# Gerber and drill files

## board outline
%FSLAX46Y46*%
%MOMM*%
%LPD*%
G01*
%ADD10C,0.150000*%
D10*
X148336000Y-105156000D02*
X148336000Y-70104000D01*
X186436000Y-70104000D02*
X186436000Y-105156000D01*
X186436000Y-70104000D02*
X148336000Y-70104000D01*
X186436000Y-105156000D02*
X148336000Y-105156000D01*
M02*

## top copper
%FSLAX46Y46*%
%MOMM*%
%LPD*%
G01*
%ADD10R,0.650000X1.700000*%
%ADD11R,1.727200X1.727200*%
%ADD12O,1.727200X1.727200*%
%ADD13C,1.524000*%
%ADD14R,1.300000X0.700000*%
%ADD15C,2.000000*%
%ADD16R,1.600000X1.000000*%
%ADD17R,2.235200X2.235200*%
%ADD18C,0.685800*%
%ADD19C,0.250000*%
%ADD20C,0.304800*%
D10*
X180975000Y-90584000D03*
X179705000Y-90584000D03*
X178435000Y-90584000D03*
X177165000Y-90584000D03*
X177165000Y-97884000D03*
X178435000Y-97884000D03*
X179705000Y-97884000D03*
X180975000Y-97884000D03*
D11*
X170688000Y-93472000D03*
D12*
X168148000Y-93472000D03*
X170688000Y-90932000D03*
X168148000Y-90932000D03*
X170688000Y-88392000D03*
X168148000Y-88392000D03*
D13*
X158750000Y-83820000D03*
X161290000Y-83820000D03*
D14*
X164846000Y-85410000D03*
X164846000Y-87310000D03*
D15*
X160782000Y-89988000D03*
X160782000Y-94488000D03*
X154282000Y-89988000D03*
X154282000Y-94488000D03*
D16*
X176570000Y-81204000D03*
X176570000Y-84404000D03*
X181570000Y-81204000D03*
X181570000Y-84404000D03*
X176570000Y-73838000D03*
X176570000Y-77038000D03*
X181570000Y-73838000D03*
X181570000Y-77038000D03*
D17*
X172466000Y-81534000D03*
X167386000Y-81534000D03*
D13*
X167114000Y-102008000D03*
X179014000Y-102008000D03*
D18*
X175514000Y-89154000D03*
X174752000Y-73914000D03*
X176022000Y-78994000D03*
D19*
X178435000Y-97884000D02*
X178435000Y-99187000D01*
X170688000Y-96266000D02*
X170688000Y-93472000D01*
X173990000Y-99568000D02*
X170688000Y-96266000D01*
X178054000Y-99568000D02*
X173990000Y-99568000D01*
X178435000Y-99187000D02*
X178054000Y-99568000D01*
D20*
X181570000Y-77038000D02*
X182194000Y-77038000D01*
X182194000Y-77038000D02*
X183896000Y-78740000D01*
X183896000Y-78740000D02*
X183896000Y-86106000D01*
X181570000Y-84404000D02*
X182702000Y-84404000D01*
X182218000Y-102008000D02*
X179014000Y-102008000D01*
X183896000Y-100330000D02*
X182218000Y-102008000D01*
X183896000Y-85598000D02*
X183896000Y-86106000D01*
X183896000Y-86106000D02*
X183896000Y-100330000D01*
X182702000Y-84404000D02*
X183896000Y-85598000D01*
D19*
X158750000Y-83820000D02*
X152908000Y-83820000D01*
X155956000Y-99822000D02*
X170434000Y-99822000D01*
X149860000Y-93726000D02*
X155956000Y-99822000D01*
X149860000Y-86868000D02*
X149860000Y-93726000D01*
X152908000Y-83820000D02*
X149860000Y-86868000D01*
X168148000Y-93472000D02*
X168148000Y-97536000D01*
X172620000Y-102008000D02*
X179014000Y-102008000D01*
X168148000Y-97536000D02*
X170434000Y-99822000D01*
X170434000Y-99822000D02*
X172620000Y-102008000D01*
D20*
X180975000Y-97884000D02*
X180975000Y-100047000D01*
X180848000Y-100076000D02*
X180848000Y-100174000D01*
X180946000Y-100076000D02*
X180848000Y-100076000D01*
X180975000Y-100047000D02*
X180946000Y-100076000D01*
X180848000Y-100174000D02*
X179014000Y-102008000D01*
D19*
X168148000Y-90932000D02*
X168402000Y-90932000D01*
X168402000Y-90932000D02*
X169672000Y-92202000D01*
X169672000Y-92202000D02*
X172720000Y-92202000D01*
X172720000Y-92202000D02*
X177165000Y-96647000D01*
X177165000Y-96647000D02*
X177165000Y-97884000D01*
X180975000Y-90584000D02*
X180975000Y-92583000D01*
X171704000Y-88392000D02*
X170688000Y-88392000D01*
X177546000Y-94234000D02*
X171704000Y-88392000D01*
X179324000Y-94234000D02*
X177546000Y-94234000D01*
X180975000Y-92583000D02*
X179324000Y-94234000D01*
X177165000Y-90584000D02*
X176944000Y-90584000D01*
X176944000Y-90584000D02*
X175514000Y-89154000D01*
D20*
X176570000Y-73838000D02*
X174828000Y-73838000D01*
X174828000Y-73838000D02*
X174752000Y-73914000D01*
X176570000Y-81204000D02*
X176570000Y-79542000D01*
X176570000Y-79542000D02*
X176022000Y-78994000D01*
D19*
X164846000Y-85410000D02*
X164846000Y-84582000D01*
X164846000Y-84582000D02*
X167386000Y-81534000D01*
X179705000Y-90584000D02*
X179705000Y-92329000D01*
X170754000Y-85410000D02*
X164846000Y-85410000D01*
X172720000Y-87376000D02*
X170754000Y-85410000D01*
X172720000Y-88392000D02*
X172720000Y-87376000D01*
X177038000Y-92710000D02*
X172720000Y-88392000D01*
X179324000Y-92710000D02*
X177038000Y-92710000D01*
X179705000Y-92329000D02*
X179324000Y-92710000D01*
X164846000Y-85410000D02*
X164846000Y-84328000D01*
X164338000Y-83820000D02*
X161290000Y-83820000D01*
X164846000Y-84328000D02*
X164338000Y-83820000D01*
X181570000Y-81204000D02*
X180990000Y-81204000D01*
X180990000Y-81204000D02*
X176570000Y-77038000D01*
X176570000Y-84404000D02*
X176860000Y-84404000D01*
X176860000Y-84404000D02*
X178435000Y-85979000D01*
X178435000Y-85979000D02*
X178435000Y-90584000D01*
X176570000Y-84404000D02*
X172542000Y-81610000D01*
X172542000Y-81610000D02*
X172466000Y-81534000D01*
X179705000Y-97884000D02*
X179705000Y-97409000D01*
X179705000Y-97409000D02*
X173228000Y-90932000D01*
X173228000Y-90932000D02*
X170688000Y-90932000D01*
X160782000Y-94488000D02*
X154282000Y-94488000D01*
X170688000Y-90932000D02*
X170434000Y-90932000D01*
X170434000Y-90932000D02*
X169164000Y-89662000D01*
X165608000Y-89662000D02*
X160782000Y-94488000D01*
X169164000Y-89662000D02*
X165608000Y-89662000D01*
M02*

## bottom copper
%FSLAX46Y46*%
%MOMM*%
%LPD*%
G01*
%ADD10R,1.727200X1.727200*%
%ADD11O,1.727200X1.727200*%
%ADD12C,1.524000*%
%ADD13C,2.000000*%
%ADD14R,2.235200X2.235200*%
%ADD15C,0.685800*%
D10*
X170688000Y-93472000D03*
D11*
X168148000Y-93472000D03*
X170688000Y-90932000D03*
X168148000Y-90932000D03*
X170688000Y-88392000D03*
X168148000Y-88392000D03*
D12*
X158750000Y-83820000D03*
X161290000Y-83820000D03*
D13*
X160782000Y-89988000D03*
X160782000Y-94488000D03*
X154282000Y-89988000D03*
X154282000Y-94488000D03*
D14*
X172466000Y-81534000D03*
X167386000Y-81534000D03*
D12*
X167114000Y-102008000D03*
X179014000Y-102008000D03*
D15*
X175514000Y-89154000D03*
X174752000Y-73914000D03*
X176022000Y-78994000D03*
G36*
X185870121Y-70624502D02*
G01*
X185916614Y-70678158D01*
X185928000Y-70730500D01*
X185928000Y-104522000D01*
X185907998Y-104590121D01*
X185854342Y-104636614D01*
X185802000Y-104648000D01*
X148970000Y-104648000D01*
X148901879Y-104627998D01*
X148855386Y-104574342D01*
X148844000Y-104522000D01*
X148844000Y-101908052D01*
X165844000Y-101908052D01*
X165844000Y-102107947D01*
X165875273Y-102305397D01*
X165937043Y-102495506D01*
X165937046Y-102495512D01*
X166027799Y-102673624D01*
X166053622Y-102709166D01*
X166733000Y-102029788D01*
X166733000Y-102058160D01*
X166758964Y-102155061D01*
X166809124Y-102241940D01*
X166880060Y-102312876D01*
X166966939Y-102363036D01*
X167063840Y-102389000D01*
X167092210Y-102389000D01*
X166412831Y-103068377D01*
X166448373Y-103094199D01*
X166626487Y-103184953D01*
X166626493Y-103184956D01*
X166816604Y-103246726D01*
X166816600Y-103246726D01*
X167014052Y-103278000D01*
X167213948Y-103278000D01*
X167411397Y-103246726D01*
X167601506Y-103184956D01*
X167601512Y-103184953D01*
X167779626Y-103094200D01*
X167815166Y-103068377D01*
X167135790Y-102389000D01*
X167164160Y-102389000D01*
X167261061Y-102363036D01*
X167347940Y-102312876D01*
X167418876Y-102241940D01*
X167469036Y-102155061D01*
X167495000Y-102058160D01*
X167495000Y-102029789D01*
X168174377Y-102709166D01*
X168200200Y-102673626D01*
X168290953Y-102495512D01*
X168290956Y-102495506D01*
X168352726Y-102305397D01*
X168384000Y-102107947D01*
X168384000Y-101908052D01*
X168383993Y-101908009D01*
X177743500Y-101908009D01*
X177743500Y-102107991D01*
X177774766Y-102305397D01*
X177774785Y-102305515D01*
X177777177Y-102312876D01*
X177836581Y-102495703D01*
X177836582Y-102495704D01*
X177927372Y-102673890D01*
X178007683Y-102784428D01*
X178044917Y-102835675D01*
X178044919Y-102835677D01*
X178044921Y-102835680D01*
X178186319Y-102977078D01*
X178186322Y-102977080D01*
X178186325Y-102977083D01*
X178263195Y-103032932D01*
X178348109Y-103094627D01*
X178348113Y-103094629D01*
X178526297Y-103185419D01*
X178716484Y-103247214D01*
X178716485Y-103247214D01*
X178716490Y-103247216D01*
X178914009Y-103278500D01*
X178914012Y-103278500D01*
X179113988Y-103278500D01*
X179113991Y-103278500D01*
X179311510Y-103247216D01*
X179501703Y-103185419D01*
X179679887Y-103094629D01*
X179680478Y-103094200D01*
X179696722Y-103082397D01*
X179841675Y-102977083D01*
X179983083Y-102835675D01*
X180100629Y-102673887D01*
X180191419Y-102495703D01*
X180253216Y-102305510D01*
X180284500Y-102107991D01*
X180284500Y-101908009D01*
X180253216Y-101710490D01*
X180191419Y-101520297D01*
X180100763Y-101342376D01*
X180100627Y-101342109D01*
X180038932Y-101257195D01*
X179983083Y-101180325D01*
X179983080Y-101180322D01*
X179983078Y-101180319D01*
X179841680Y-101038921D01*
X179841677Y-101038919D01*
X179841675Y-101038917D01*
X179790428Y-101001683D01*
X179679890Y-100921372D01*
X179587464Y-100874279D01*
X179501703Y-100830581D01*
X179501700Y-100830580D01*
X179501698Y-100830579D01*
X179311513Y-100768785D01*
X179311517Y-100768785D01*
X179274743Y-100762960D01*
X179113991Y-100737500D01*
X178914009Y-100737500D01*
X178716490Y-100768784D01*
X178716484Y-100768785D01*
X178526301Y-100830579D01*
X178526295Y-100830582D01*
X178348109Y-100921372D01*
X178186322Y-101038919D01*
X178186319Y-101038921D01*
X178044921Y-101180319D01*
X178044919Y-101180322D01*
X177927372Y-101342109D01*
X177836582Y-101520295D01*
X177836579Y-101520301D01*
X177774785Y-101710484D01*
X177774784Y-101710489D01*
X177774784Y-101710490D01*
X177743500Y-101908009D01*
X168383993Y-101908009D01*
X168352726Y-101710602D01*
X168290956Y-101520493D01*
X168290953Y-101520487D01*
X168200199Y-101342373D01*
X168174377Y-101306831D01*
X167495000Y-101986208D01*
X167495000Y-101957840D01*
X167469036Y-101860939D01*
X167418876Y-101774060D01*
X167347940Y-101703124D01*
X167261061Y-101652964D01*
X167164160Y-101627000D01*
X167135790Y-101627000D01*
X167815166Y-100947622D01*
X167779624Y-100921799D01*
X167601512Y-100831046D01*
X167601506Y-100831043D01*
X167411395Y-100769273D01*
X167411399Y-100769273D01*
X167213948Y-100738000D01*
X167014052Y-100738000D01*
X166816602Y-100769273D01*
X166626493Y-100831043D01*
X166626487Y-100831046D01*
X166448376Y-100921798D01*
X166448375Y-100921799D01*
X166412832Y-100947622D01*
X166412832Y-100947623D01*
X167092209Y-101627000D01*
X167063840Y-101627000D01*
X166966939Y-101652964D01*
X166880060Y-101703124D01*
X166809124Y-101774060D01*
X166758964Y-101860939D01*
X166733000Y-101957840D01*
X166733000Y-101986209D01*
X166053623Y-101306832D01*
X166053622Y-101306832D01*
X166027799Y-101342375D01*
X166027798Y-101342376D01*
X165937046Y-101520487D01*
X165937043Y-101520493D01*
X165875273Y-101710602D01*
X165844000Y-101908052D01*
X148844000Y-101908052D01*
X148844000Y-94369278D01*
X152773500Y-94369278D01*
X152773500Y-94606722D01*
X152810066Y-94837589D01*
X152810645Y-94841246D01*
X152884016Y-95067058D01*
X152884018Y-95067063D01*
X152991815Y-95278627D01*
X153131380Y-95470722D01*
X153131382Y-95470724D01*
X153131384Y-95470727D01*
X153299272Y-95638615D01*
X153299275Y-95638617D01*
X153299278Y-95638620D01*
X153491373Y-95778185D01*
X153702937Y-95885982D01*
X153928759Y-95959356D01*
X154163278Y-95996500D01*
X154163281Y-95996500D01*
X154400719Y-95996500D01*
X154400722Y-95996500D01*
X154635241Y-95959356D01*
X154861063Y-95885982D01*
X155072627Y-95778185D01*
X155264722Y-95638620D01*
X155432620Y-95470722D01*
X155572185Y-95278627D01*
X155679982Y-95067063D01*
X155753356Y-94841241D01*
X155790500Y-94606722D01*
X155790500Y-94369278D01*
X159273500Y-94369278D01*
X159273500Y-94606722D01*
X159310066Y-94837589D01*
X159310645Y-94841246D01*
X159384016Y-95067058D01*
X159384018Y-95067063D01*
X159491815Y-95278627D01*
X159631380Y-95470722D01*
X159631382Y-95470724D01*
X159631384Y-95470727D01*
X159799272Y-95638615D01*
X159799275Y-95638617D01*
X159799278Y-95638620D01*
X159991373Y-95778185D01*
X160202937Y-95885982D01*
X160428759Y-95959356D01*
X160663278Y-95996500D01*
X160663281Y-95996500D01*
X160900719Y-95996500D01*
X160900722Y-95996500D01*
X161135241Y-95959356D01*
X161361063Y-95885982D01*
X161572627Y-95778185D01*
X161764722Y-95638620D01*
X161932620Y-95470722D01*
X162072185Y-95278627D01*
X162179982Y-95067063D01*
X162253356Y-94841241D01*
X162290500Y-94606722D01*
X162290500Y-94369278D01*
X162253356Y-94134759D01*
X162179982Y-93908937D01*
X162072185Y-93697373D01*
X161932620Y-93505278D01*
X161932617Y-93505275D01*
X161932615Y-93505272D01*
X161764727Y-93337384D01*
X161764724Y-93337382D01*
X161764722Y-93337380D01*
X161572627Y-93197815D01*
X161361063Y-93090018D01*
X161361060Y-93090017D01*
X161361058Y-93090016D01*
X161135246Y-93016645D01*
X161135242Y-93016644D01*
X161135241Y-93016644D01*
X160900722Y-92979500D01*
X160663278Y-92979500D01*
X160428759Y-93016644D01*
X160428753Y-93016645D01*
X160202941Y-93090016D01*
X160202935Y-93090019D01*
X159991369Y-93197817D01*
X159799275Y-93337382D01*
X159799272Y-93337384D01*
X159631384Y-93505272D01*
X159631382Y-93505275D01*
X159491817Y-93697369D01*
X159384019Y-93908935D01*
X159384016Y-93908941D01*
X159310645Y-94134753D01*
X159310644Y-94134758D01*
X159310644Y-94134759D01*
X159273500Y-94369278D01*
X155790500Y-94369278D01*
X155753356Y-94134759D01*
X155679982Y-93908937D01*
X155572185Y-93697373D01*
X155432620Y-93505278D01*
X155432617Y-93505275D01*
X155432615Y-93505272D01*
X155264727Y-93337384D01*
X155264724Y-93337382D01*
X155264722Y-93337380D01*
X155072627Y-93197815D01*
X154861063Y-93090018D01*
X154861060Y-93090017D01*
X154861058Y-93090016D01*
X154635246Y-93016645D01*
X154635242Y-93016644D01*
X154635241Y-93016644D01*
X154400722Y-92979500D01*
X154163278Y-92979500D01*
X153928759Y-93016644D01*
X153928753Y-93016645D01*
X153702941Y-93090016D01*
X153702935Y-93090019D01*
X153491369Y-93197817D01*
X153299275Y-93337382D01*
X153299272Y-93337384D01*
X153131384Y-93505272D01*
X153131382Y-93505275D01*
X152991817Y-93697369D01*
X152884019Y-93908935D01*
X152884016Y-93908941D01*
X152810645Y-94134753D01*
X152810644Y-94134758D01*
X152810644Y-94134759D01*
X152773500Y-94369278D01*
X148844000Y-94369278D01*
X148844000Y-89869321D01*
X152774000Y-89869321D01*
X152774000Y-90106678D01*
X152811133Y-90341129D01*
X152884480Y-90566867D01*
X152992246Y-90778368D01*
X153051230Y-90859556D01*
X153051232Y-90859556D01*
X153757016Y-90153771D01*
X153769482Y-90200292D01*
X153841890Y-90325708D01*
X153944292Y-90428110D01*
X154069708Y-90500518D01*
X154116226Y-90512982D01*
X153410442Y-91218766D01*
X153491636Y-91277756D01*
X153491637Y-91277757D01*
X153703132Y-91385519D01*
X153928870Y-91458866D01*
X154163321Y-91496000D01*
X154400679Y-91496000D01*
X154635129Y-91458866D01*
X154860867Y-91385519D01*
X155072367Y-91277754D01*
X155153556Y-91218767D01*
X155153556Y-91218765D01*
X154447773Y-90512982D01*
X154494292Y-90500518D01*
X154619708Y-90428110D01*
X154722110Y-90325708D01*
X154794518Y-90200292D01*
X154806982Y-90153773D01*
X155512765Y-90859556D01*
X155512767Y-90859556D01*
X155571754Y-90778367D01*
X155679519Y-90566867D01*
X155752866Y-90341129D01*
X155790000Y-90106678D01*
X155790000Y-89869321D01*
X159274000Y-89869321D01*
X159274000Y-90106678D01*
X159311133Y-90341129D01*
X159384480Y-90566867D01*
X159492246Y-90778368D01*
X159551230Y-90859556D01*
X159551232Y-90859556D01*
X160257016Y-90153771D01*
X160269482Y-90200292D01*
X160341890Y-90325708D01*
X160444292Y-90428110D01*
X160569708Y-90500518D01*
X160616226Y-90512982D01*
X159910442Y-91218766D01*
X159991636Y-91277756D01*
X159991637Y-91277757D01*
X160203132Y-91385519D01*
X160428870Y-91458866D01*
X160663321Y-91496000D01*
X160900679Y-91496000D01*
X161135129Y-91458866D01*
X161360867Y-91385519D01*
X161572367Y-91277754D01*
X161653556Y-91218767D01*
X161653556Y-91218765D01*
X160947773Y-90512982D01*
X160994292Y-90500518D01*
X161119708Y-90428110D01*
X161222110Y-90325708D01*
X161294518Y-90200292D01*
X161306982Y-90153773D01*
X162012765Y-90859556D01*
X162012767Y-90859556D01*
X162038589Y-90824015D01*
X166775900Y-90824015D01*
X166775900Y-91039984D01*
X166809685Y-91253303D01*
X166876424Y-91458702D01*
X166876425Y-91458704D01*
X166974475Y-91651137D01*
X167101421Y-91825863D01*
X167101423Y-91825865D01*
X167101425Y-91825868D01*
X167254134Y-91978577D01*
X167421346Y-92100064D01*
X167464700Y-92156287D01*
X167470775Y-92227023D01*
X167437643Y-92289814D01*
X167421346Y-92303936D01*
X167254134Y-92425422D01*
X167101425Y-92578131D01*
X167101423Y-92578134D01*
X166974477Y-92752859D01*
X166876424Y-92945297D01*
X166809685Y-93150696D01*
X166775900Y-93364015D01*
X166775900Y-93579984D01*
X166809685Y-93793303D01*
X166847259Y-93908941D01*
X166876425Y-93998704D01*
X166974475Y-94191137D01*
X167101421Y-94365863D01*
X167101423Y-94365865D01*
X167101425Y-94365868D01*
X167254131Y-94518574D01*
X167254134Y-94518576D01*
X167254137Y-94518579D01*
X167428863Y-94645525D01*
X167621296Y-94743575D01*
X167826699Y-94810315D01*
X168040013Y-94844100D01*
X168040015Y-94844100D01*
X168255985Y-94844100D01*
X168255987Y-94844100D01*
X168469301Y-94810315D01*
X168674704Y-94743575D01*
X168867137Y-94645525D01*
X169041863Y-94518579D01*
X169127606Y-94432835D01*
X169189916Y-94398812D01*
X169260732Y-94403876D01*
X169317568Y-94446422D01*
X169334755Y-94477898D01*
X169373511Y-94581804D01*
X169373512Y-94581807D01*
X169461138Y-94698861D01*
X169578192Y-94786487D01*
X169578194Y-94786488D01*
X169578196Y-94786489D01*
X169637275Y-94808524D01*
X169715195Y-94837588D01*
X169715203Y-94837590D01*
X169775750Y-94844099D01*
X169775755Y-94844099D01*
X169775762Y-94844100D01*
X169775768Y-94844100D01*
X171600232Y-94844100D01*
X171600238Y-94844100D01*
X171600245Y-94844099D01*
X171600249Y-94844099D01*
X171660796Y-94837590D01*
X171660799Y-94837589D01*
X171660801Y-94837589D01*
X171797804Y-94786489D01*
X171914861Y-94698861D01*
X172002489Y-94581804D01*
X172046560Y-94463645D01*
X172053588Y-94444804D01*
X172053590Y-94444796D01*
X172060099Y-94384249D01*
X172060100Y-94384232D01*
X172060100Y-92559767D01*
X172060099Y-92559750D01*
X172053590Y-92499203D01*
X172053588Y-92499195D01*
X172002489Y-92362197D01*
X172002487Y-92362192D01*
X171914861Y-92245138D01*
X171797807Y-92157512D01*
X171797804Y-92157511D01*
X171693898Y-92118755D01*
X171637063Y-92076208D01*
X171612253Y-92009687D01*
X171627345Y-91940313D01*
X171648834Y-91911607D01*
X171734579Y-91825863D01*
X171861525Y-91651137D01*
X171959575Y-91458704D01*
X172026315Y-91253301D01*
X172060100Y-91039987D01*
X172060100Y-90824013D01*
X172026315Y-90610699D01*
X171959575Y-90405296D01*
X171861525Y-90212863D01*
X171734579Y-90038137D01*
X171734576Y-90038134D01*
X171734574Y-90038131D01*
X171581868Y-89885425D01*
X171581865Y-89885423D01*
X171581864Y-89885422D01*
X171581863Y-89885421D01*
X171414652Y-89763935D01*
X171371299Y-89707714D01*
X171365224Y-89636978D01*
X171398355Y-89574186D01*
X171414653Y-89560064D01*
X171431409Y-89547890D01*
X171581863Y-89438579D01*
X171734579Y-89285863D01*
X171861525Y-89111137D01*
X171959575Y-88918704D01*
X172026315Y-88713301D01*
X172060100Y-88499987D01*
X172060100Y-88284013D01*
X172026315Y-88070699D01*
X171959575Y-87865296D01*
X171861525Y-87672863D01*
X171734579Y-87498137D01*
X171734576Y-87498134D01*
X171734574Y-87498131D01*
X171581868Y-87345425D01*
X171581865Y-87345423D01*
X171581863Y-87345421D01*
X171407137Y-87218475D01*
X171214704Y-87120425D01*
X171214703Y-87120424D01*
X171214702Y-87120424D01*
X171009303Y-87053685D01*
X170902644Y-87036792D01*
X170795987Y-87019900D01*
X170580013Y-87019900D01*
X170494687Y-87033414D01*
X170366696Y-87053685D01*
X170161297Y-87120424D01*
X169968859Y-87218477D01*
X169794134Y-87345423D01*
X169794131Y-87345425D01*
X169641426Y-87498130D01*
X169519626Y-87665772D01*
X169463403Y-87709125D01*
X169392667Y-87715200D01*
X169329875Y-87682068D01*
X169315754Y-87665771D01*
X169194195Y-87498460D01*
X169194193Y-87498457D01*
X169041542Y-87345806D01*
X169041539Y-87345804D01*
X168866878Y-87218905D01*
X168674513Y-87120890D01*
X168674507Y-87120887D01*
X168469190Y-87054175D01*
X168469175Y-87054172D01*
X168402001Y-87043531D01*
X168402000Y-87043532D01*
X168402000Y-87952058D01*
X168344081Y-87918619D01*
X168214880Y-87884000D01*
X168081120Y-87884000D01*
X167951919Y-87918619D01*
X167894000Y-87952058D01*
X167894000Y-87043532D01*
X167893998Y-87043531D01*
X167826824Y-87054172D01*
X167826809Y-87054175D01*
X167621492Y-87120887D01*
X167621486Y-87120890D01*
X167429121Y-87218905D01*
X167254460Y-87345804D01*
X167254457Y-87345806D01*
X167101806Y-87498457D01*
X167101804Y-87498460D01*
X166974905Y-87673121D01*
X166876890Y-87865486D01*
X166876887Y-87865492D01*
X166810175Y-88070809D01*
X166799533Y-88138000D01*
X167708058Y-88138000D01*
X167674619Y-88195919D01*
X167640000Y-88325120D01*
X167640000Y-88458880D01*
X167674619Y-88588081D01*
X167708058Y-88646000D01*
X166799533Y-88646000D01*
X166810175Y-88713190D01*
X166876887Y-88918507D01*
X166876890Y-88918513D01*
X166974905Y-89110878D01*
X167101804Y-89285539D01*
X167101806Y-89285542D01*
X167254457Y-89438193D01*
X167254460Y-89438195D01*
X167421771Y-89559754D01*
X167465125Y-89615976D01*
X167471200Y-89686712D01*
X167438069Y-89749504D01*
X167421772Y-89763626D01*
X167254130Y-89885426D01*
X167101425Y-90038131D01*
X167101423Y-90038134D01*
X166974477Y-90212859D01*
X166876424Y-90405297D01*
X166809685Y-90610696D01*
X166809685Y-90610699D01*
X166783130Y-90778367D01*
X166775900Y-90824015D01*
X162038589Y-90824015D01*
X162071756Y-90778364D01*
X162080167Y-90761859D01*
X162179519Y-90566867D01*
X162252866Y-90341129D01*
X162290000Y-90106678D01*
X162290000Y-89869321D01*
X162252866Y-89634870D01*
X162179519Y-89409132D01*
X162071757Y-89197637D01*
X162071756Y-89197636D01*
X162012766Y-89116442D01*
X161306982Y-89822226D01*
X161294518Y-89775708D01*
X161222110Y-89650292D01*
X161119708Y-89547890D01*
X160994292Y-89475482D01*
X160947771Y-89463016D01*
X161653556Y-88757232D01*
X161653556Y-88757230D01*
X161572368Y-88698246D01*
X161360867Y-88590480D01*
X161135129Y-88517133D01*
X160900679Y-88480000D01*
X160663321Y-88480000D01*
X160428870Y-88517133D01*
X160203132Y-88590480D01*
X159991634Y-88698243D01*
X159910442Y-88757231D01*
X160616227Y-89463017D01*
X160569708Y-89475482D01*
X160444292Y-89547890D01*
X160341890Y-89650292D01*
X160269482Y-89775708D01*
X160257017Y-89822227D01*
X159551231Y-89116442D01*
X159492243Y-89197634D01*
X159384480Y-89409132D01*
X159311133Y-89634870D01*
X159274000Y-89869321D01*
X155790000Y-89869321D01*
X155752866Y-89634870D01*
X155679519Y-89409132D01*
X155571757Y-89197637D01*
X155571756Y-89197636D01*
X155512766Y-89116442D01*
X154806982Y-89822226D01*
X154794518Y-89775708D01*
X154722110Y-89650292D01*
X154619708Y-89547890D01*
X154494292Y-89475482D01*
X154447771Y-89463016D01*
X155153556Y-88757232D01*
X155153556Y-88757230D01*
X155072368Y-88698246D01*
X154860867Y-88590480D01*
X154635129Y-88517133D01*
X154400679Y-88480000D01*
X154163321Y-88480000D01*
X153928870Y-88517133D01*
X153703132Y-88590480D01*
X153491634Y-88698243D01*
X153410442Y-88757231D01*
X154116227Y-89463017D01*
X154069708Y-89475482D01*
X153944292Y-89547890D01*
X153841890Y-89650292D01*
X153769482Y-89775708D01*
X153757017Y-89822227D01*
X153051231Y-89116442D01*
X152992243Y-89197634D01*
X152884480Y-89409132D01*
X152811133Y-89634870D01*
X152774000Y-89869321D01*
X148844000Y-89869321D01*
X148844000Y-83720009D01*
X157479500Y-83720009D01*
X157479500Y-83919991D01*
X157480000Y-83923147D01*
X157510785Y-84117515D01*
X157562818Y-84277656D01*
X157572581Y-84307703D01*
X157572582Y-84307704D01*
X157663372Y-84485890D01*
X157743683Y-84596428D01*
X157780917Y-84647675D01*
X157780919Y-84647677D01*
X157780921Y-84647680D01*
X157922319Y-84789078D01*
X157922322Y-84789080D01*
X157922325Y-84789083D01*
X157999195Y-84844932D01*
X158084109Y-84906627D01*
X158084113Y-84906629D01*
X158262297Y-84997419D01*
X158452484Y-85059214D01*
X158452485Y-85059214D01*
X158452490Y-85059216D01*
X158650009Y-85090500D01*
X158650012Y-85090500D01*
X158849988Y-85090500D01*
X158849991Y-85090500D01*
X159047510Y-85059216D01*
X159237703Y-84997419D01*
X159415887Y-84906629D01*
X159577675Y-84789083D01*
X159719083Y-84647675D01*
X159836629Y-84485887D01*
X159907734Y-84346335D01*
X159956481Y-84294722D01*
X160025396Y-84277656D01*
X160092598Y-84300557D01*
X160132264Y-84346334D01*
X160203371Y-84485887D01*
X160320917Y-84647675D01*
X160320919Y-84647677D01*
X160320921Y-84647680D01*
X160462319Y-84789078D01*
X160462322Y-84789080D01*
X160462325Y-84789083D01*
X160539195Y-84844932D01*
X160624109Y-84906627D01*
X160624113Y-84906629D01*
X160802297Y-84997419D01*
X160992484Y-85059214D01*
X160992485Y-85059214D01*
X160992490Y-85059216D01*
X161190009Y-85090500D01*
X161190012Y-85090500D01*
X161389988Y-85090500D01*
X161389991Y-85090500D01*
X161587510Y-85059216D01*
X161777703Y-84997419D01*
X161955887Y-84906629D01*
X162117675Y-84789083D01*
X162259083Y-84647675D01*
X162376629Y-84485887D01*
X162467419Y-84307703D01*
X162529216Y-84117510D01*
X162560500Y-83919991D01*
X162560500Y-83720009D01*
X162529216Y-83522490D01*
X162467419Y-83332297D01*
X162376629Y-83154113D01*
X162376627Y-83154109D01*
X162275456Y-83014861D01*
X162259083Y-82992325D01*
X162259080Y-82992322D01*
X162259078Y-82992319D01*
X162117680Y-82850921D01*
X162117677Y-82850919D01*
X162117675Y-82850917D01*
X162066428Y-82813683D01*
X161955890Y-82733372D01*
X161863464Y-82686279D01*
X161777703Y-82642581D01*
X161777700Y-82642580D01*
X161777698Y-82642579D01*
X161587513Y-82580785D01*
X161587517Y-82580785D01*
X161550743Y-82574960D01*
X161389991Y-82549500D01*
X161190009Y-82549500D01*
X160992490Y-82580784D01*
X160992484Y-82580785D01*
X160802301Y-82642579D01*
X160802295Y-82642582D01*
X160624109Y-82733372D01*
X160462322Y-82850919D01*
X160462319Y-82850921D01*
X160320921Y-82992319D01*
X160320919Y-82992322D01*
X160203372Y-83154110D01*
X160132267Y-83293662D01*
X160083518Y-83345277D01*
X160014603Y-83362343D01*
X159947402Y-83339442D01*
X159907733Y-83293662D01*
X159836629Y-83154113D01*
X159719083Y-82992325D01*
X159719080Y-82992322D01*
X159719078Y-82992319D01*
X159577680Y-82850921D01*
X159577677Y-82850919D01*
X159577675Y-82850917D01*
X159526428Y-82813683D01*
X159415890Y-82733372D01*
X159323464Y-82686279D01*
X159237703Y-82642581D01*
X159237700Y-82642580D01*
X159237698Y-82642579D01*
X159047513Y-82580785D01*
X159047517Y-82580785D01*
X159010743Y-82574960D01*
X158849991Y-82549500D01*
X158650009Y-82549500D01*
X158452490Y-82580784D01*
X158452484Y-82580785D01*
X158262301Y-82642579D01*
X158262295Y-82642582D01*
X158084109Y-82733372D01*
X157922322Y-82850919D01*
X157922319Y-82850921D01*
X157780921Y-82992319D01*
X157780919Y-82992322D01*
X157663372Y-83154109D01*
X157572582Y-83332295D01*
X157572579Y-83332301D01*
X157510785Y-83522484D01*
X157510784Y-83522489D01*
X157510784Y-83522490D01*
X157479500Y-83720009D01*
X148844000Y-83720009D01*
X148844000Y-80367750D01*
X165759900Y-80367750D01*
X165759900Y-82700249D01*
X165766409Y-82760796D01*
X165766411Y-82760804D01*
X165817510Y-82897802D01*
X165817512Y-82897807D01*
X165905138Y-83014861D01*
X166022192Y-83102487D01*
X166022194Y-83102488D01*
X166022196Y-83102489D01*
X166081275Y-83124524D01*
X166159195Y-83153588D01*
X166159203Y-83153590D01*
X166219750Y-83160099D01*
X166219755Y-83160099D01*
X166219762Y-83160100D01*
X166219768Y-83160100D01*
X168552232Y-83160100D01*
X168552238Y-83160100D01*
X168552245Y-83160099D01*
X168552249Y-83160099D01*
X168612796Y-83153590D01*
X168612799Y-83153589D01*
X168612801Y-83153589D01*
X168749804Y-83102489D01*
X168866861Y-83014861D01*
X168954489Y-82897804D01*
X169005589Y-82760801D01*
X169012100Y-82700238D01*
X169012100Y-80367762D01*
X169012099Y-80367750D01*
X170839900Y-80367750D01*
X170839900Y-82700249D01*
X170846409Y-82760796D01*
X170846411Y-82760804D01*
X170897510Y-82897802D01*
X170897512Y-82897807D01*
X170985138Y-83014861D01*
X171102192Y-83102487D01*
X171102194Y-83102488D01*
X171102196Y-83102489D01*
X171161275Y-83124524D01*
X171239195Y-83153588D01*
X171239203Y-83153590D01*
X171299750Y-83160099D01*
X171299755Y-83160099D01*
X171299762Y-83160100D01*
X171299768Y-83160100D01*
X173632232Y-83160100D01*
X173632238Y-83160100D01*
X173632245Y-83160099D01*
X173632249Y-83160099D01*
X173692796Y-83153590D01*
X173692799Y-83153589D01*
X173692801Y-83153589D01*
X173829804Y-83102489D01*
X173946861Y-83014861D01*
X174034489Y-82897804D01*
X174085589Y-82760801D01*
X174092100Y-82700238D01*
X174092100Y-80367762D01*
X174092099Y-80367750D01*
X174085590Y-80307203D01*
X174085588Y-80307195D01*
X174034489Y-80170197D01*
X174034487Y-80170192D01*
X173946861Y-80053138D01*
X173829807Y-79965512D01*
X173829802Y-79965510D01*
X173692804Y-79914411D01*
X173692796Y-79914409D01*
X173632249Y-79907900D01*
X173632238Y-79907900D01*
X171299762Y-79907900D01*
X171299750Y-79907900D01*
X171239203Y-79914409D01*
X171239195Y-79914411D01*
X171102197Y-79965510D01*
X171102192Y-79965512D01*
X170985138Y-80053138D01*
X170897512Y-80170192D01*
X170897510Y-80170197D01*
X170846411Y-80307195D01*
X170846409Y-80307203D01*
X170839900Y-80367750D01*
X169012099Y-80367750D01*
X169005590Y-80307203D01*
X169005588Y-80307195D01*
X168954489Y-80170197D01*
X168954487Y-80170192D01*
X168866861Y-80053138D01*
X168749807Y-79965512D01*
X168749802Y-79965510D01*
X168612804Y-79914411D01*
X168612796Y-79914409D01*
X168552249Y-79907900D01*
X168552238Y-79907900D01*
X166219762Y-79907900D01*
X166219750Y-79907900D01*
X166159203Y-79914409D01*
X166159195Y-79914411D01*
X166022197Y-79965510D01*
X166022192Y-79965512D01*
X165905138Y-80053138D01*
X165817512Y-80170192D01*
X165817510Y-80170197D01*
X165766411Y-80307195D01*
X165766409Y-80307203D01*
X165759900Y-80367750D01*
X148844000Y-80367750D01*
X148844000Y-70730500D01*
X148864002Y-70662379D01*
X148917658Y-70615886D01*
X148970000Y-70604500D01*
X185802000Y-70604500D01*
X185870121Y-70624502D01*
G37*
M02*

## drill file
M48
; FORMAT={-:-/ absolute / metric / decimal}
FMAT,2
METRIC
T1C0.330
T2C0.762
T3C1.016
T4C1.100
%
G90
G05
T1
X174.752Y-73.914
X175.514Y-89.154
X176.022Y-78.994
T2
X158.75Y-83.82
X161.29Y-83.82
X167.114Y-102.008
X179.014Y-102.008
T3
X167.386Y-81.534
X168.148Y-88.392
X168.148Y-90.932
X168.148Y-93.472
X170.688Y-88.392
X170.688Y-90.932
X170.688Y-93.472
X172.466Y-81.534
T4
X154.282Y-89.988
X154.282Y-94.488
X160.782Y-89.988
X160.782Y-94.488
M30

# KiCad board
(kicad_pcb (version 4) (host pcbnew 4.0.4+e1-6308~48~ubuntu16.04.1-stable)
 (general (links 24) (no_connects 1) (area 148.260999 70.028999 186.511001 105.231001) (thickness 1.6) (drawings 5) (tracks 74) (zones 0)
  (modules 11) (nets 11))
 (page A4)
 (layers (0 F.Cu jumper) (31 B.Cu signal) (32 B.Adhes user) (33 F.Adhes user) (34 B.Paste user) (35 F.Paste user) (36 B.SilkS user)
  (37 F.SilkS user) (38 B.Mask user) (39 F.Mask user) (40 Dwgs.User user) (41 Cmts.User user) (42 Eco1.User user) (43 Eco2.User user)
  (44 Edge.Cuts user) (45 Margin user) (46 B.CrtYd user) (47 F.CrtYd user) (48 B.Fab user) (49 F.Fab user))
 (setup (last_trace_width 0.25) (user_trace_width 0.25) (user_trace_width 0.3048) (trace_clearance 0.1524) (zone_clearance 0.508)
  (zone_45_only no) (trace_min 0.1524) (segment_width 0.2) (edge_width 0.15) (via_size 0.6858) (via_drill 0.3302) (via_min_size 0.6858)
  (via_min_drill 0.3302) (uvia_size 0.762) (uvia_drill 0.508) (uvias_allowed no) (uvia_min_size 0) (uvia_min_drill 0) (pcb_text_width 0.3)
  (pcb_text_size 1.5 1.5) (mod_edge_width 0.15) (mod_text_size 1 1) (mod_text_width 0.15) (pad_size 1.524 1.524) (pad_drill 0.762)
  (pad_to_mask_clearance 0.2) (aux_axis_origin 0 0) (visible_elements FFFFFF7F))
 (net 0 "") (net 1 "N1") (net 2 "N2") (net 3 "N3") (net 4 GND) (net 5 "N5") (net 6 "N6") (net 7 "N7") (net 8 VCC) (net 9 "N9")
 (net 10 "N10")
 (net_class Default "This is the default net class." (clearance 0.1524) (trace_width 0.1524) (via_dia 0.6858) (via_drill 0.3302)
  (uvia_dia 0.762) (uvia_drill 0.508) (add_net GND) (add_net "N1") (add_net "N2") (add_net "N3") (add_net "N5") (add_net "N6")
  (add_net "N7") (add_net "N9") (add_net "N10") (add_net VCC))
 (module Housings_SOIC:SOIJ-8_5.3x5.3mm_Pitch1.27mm (layer F.Cu) (at 179.07 94.234 270)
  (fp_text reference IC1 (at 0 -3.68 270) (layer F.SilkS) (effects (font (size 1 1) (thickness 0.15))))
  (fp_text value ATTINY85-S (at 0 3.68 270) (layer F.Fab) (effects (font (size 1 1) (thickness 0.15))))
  (pad 1 smd rect (at -3.65 -1.905 270) (size 1.7 0.65) (layers F.Cu F.Paste F.Mask) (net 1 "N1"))
  (pad 2 smd rect (at -3.65 -0.635 270) (size 1.7 0.65) (layers F.Cu F.Paste F.Mask) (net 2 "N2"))
  (pad 3 smd rect (at -3.65 0.635 270) (size 1.7 0.65) (layers F.Cu F.Paste F.Mask) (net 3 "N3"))
  (pad 4 smd rect (at -3.65 1.905 270) (size 1.7 0.65) (layers F.Cu F.Paste F.Mask) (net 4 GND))
  (pad 5 smd rect (at 3.65 1.905 270) (size 1.7 0.65) (layers F.Cu F.Paste F.Mask) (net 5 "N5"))
  (pad 6 smd rect (at 3.65 0.635 270) (size 1.7 0.65) (layers F.Cu F.Paste F.Mask) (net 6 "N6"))
  (pad 7 smd rect (at 3.65 -0.635 270) (size 1.7 0.65) (layers F.Cu F.Paste F.Mask) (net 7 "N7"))
  (pad 8 smd rect (at 3.65 -1.905 270) (size 1.7 0.65) (layers F.Cu F.Paste F.Mask) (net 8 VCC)))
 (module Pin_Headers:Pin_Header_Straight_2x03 (layer F.Cu) (at 170.688 93.472 180)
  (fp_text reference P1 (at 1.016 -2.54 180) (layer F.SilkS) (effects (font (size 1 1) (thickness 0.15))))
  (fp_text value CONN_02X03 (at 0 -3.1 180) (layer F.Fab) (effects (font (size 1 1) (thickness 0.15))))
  (pad 1 thru_hole rect (at 0 0 180) (size 1.7272 1.7272) (drill 1.016) (layers *.Cu *.Mask F.SilkS) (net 6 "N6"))
  (pad 2 thru_hole oval (at 2.54 0 180) (size 1.7272 1.7272) (drill 1.016) (layers *.Cu *.Mask F.SilkS) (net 8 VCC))
  (pad 3 thru_hole oval (at 0 2.54 180) (size 1.7272 1.7272) (drill 1.016) (layers *.Cu *.Mask F.SilkS) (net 7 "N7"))
  (pad 4 thru_hole oval (at 2.54 2.54 180) (size 1.7272 1.7272) (drill 1.016) (layers *.Cu *.Mask F.SilkS) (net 5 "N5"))
  (pad 5 thru_hole oval (at 0 5.08 180) (size 1.7272 1.7272) (drill 1.016) (layers *.Cu *.Mask F.SilkS) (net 1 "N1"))
  (pad 6 thru_hole oval (at 2.54 5.08 180) (size 1.7272 1.7272) (drill 1.016) (layers *.Cu *.Mask F.SilkS) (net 4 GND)))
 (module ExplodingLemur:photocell (layer F.Cu) (at 160.02 83.82)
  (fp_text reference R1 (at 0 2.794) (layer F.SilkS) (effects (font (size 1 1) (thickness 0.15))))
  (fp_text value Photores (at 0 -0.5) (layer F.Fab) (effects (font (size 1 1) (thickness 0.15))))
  (pad 1 thru_hole circle (at -1.27 0) (size 1.524 1.524) (drill 0.762) (layers *.Cu *.Mask) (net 8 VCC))
  (pad 2 thru_hole circle (at 1.27 0) (size 1.524 1.524) (drill 0.762) (layers *.Cu *.Mask) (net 2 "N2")))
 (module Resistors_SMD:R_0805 (layer F.Cu) (at 164.846 86.36 270)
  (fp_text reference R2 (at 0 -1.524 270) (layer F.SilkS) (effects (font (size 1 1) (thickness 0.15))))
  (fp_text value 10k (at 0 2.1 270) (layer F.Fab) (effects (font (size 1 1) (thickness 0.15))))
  (pad 1 smd rect (at -0.95 0 270) (size 0.7 1.3) (layers F.Cu F.Paste F.Mask) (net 2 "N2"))
  (pad 2 smd rect (at 0.95 0 270) (size 0.7 1.3) (layers F.Cu F.Paste F.Mask) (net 4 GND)))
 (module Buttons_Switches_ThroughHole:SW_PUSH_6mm (layer F.Cu) (at 160.782 94.488 180)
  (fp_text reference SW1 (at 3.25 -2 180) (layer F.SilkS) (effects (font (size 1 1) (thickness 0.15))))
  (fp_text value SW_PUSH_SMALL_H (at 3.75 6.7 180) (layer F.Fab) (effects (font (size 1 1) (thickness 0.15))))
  (pad 2 thru_hole circle (at 0 4.5 270) (size 2 2) (drill 1.1) (layers *.Cu *.Mask) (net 4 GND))
  (pad 1 thru_hole circle (at 0 0 270) (size 2 2) (drill 1.1) (layers *.Cu *.Mask) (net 7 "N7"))
  (pad 2 thru_hole circle (at 6.5 4.5 270) (size 2 2) (drill 1.1) (layers *.Cu *.Mask) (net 4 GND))
  (pad 1 thru_hole circle (at 6.5 0 270) (size 2 2) (drill 1.1) (layers *.Cu *.Mask) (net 7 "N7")))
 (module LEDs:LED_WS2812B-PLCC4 (layer F.Cu) (at 179.07 82.804 180)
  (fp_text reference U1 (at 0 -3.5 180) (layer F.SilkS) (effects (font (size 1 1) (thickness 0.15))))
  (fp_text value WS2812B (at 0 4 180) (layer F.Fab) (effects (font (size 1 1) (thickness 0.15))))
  (pad 3 smd rect (at 2.5 1.6 180) (size 1.6 1) (layers F.Cu F.Paste F.Mask) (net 4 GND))
  (pad 4 smd rect (at 2.5 -1.6 180) (size 1.6 1) (layers F.Cu F.Paste F.Mask) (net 3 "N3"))
  (pad 2 smd rect (at -2.5 1.6 180) (size 1.6 1) (layers F.Cu F.Paste F.Mask) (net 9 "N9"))
  (pad 1 smd rect (at -2.5 -1.6 180) (size 1.6 1) (layers F.Cu F.Paste F.Mask) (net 8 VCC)))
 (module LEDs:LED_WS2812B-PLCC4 (layer F.Cu) (at 179.07 75.438 180)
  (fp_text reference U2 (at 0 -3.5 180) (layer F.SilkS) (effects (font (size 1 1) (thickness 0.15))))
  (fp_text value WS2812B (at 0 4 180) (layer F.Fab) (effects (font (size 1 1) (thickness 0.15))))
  (pad 3 smd rect (at 2.5 1.6 180) (size 1.6 1) (layers F.Cu F.Paste F.Mask) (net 4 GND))
  (pad 4 smd rect (at 2.5 -1.6 180) (size 1.6 1) (layers F.Cu F.Paste F.Mask) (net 9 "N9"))
  (pad 2 smd rect (at -2.5 1.6 180) (size 1.6 1) (layers F.Cu F.Paste F.Mask) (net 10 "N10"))
  (pad 1 smd rect (at -2.5 -1.6 180) (size 1.6 1) (layers F.Cu F.Paste F.Mask) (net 8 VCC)))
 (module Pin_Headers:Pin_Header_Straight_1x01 (layer F.Cu) (at 172.466 81.534)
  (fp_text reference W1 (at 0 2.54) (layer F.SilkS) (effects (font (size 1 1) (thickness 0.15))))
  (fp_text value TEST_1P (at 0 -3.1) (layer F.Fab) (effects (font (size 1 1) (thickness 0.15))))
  (pad 1 thru_hole rect (at 0 0) (size 2.2352 2.2352) (drill 1.016) (layers *.Cu *.Mask F.SilkS) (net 3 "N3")))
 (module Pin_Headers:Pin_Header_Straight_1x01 (layer F.Cu) (at 167.386 81.534)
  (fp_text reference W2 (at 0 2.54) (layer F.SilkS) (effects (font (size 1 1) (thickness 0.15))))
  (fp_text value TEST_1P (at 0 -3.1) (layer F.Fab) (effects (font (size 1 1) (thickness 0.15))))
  (pad 1 thru_hole rect (at 0 0) (size 2.2352 2.2352) (drill 1.016) (layers *.Cu *.Mask F.SilkS) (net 2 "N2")))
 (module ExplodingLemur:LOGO (layer B.Cu) (at 182.88 73.406 180)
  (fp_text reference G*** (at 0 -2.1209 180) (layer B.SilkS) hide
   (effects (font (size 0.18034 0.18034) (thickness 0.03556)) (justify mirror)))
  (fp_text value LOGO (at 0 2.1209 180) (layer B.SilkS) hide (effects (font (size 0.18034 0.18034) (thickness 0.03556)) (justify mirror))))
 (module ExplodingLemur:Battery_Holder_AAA (layer B.Cu) (at 148.844 104.648)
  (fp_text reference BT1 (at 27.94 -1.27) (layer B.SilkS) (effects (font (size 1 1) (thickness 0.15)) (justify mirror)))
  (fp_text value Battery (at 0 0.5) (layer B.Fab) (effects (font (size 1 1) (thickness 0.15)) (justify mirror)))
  (pad 2 thru_hole circle (at 18.27 -2.64) (size 1.524 1.524) (drill 0.762) (layers *.Cu *.Mask) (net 4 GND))
  (pad 1 thru_hole circle (at 30.17 -2.64) (size 1.524 1.524) (drill 0.762) (layers *.Cu *.Mask) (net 8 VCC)))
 (gr_line (start 148.336 105.156) (end 148.336 70.104) (angle 90) (layer Edge.Cuts) (width 0.15))
 (gr_line (start 186.436 70.104) (end 186.436 105.156) (angle 90) (layer Edge.Cuts) (width 0.15))
 (gr_line (start 186.436 70.104) (end 148.336 70.104) (angle 90) (layer Edge.Cuts) (width 0.15))
 (gr_line (start 186.436 105.156) (end 148.336 105.156) (angle 90) (layer Edge.Cuts) (width 0.15))
 (segment (start 178.435 97.884) (end 178.435 99.187) (width 0.25) (layer F.Cu) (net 6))
 (segment (start 170.688 96.266) (end 170.688 93.472) (width 0.25) (layer F.Cu) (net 6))
 (segment (start 173.99 99.568) (end 170.688 96.266) (width 0.25) (layer F.Cu) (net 6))
 (segment (start 178.054 99.568) (end 173.99 99.568) (width 0.25) (layer F.Cu) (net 6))
 (segment (start 178.435 99.187) (end 178.054 99.568) (width 0.25) (layer F.Cu) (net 6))
 (segment (start 181.57 77.038) (end 182.194 77.038) (width 0.3048) (layer F.Cu) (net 8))
 (segment (start 182.194 77.038) (end 183.896 78.74) (width 0.3048) (layer F.Cu) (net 8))
 (segment (start 183.896 78.74) (end 183.896 86.106) (width 0.3048) (layer F.Cu) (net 8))
 (segment (start 181.57 84.404) (end 182.702 84.404) (width 0.3048) (layer F.Cu) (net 8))
 (segment (start 182.218 102.008) (end 179.014 102.008) (width 0.3048) (layer F.Cu) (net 8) (status 20))
 (segment (start 183.896 100.33) (end 182.218 102.008) (width 0.3048) (layer F.Cu) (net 8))
 (segment (start 183.896 85.598) (end 183.896 86.106) (width 0.3048) (layer F.Cu) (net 8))
 (segment (start 183.896 86.106) (end 183.896 100.33) (width 0.3048) (layer F.Cu) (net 8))
 (segment (start 182.702 84.404) (end 183.896 85.598) (width 0.3048) (layer F.Cu) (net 8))
 (segment (start 158.75 83.82) (end 152.908 83.82) (width 0.25) (layer F.Cu) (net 8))
 (segment (start 155.956 99.822) (end 170.434 99.822) (width 0.25) (layer F.Cu) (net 8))
 (segment (start 149.86 93.726) (end 155.956 99.822) (width 0.25) (layer F.Cu) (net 8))
 (segment (start 149.86 86.868) (end 149.86 93.726) (width 0.25) (layer F.Cu) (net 8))
 (segment (start 152.908 83.82) (end 149.86 86.868) (width 0.25) (layer F.Cu) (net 8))
 (segment (start 168.148 93.472) (end 168.148 97.536) (width 0.25) (layer F.Cu) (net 8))
 (segment (start 172.62 102.008) (end 179.014 102.008) (width 0.25) (layer F.Cu) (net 8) (status 20))
 (segment (start 168.148 97.536) (end 170.434 99.822) (width 0.25) (layer F.Cu) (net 8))
 (segment (start 170.434 99.822) (end 172.62 102.008) (width 0.25) (layer F.Cu) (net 8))
 (segment (start 180.975 97.884) (end 180.975 100.047) (width 0.3048) (layer F.Cu) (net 8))
 (segment (start 180.848 100.076) (end 180.848 100.174) (width 0.3048) (layer F.Cu) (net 8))
 (segment (start 180.946 100.076) (end 180.848 100.076) (width 0.3048) (layer F.Cu) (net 8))
 (segment (start 180.975 100.047) (end 180.946 100.076) (width 0.3048) (layer F.Cu) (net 8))
 (segment (start 180.848 100.174) (end 179.014 102.008) (width 0.3048) (layer F.Cu) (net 8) (status 20))
 (segment (start 168.148 90.932) (end 168.402 90.932) (width 0.25) (layer F.Cu) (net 5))
 (segment (start 168.402 90.932) (end 169.672 92.202) (width 0.25) (layer F.Cu) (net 5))
 (segment (start 169.672 92.202) (end 172.72 92.202) (width 0.25) (layer F.Cu) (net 5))
 (segment (start 172.72 92.202) (end 177.165 96.647) (width 0.25) (layer F.Cu) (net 5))
 (segment (start 177.165 96.647) (end 177.165 97.884) (width 0.25) (layer F.Cu) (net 5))
 (segment (start 180.975 90.584) (end 180.975 92.583) (width 0.25) (layer F.Cu) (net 1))
 (segment (start 171.704 88.392) (end 170.688 88.392) (width 0.25) (layer F.Cu) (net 1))
 (segment (start 177.546 94.234) (end 171.704 88.392) (width 0.25) (layer F.Cu) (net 1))
 (segment (start 179.324 94.234) (end 177.546 94.234) (width 0.25) (layer F.Cu) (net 1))
 (segment (start 180.975 92.583) (end 179.324 94.234) (width 0.25) (layer F.Cu) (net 1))
 (segment (start 177.165 90.584) (end 176.944 90.584) (width 0.25) (layer F.Cu) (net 4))
 (segment (start 176.944 90.584) (end 175.514 89.154) (width 0.25) (layer F.Cu) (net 4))
 (via (at 175.514 89.154) (size 0.6858) (drill 0.3302) (layers F.Cu B.Cu) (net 4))
 (segment (start 176.57 73.838) (end 174.828 73.838) (width 0.3048) (layer F.Cu) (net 4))
 (via (at 174.752 73.914) (size 0.6858) (drill 0.3302) (layers F.Cu B.Cu) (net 4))
 (segment (start 174.828 73.838) (end 174.752 73.914) (width 0.3048) (layer F.Cu) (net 4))
 (segment (start 176.57 81.204) (end 176.57 79.542) (width 0.3048) (layer F.Cu) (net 4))
 (via (at 176.022 78.994) (size 0.6858) (drill 0.3302) (layers F.Cu B.Cu) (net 4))
 (segment (start 176.57 79.542) (end 176.022 78.994) (width 0.3048) (layer F.Cu) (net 4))
 (segment (start 164.846 85.41) (end 164.846 84.582) (width 0.25) (layer F.Cu) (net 2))
 (segment (start 164.846 84.582) (end 167.386 81.534) (width 0.25) (layer F.Cu) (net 2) (status 20))
 (segment (start 179.705 90.584) (end 179.705 92.329) (width 0.25) (layer F.Cu) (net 2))
 (segment (start 170.754 85.41) (end 164.846 85.41) (width 0.25) (layer F.Cu) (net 2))
 (segment (start 172.72 87.376) (end 170.754 85.41) (width 0.25) (layer F.Cu) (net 2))
 (segment (start 172.72 88.392) (end 172.72 87.376) (width 0.25) (layer F.Cu) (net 2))
 (segment (start 177.038 92.71) (end 172.72 88.392) (width 0.25) (layer F.Cu) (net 2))
 (segment (start 179.324 92.71) (end 177.038 92.71) (width 0.25) (layer F.Cu) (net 2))
 (segment (start 179.705 92.329) (end 179.324 92.71) (width 0.25) (layer F.Cu) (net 2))
 (segment (start 164.846 85.41) (end 164.846 84.328) (width 0.25) (layer F.Cu) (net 2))
 (segment (start 164.338 83.82) (end 161.29 83.82) (width 0.25) (layer F.Cu) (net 2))
 (segment (start 164.846 84.328) (end 164.338 83.82) (width 0.25) (layer F.Cu) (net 2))
 (segment (start 181.57 81.204) (end 180.99 81.204) (width 0.25) (layer F.Cu) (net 9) (status 30))
 (segment (start 180.99 81.204) (end 176.57 77.038) (width 0.25) (layer F.Cu) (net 9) (status 20))
 (segment (start 176.57 84.404) (end 176.86 84.404) (width 0.25) (layer F.Cu) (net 3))
 (segment (start 176.86 84.404) (end 178.435 85.979) (width 0.25) (layer F.Cu) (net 3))
 (segment (start 178.435 85.979) (end 178.435 90.584) (width 0.25) (layer F.Cu) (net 3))
 (segment (start 176.57 84.404) (end 172.542 81.61) (width 0.25) (layer F.Cu) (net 3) (status 20))
 (segment (start 172.542 81.61) (end 172.466 81.534) (width 0.25) (layer F.Cu) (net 3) (status 30))
 (segment (start 179.705 97.884) (end 179.705 97.409) (width 0.25) (layer F.Cu) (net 7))
 (segment (start 179.705 97.409) (end 173.228 90.932) (width 0.25) (layer F.Cu) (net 7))
 (segment (start 173.228 90.932) (end 170.688 90.932) (width 0.25) (layer F.Cu) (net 7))
 (segment (start 160.782 94.488) (end 154.282 94.488) (width 0.25) (layer F.Cu) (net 7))
 (segment (start 170.688 90.932) (end 170.434 90.932) (width 0.25) (layer F.Cu) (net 7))
 (segment (start 170.434 90.932) (end 169.164 89.662) (width 0.25) (layer F.Cu) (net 7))
 (segment (start 165.608 89.662) (end 160.782 94.488) (width 0.25) (layer F.Cu) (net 7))
 (segment (start 169.164 89.662) (end 165.608 89.662) (width 0.25) (layer F.Cu) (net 7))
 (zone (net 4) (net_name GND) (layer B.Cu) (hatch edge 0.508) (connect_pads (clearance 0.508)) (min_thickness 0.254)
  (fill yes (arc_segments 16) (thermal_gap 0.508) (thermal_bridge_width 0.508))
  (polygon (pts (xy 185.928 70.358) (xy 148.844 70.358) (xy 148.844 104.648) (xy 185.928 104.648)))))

